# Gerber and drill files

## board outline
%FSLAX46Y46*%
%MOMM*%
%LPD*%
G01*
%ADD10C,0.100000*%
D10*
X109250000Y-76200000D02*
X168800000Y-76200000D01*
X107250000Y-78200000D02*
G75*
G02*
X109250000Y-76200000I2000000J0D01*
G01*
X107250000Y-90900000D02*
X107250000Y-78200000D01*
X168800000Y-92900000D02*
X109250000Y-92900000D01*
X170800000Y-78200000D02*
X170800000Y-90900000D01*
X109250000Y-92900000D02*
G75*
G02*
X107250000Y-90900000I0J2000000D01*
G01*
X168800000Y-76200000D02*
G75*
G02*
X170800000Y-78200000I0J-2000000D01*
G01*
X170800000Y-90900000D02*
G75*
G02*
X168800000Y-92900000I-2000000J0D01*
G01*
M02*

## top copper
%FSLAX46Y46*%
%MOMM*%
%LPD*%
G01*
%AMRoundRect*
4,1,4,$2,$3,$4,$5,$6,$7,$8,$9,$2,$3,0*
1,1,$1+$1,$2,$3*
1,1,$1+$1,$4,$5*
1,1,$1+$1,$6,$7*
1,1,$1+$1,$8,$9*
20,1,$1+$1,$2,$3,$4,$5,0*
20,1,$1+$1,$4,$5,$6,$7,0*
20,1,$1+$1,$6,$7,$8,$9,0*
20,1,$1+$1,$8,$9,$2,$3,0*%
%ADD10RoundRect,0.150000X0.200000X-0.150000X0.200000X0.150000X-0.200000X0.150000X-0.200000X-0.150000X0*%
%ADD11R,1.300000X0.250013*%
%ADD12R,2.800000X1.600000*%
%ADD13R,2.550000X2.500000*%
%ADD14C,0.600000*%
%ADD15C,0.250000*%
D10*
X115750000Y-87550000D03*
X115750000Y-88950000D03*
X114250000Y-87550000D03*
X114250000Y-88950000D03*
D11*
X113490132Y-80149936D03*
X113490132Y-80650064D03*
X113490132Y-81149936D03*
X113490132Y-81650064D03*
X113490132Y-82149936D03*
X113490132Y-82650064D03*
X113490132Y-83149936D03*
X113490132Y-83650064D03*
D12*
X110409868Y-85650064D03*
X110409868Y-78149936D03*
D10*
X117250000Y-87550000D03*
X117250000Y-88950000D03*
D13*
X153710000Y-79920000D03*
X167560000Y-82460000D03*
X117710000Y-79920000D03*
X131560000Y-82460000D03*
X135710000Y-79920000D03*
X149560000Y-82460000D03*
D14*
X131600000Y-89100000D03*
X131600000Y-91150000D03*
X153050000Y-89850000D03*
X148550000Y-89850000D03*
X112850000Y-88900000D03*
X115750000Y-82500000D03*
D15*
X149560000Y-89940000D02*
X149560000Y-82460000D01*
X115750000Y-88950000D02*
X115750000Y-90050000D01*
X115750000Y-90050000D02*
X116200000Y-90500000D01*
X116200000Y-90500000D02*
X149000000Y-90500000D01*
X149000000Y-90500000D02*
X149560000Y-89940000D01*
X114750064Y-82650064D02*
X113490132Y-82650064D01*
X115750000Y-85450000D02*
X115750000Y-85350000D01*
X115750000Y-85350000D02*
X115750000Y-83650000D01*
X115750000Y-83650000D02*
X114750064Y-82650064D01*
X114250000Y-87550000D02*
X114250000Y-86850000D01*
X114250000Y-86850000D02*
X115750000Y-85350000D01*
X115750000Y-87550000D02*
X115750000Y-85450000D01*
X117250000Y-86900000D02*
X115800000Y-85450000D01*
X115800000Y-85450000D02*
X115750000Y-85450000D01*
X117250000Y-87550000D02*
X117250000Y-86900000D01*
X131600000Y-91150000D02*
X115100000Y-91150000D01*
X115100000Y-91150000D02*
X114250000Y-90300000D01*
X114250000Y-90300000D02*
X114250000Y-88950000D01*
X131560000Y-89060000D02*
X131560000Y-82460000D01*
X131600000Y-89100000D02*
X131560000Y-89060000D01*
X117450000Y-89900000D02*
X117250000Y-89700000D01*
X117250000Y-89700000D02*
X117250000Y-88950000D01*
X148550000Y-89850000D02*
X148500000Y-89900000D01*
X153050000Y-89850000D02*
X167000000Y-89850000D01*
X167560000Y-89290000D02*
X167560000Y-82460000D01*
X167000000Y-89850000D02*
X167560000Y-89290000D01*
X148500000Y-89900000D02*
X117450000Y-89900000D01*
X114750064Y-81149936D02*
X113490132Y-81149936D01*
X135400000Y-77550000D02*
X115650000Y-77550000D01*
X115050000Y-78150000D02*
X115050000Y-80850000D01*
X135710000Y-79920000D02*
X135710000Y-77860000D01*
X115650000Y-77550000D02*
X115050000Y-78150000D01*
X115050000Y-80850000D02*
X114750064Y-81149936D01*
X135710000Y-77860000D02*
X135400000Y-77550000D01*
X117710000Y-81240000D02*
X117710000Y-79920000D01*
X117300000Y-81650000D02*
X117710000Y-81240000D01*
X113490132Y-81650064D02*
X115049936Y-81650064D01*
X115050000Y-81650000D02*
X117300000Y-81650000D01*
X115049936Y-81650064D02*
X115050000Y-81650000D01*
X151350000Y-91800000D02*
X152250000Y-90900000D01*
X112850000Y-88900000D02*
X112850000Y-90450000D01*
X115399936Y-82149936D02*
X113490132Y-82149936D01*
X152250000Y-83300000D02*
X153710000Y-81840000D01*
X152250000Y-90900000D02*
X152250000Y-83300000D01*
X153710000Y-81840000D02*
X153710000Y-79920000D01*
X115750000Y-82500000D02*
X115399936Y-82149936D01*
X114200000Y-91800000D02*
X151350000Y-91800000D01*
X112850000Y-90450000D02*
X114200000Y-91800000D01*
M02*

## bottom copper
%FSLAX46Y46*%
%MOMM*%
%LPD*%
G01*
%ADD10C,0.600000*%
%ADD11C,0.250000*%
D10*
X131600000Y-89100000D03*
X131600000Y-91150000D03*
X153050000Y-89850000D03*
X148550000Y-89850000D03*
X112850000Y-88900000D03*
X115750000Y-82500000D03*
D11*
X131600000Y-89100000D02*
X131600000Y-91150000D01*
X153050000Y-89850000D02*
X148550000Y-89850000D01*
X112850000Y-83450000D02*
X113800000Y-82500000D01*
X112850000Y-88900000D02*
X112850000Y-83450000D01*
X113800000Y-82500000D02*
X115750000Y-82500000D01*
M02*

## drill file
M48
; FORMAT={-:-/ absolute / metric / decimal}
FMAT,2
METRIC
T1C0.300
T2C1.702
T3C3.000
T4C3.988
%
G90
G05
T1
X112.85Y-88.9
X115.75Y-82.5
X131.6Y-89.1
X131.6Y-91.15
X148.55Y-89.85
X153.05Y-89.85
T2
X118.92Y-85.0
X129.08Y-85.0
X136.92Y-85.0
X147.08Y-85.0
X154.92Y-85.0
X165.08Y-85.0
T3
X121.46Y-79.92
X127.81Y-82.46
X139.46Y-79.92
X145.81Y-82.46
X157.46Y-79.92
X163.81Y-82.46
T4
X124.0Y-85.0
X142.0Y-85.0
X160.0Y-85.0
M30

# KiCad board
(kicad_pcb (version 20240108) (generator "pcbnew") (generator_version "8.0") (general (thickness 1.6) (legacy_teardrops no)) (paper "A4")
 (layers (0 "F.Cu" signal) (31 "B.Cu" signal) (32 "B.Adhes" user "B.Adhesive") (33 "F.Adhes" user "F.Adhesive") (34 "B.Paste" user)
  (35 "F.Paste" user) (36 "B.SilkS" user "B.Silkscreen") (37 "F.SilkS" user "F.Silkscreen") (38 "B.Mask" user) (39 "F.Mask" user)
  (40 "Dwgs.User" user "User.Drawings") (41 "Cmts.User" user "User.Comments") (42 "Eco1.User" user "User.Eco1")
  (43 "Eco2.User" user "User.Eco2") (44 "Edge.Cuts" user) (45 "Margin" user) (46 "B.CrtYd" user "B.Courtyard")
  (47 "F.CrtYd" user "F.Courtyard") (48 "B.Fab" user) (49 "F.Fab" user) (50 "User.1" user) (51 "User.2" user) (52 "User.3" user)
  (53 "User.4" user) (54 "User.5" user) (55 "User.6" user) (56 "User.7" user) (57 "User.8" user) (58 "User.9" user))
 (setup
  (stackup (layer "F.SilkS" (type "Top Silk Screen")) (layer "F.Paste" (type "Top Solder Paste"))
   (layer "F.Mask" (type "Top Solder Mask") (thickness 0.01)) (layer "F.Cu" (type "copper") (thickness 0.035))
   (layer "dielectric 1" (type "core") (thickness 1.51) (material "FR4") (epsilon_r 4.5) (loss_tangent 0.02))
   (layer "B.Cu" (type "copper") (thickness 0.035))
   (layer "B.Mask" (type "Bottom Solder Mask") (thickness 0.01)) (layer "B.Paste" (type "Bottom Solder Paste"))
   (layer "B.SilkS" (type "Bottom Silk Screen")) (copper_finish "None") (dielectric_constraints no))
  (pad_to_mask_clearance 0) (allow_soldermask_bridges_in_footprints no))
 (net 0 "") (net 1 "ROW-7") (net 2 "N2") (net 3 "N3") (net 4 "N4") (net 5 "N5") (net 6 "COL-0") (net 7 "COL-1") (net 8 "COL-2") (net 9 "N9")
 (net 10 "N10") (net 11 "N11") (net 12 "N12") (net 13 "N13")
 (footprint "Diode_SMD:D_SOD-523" (layer "F.Cu") (at 115.75 88.25 -90)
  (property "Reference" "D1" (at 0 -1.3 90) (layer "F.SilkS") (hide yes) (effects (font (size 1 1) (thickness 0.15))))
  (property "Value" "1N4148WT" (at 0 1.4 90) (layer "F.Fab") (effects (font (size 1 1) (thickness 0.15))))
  (pad "1" smd roundrect (at -0.7 0 90) (size 0.6 0.7) (layers "F.Cu" "F.Paste" "F.Mask") (roundrect_rratio 0.25) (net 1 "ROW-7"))
  (pad "2" smd roundrect (at 0.7 0 90) (size 0.6 0.7) (layers "F.Cu" "F.Paste" "F.Mask") (roundrect_rratio 0.25) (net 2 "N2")))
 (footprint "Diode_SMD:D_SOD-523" (layer "F.Cu") (at 114.25 88.25 -90)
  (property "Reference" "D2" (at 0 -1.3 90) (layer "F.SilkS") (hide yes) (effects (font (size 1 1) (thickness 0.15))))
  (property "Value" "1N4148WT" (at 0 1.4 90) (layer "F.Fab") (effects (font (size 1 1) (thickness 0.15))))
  (pad "1" smd roundrect (at -0.7 0 90) (size 0.6 0.7) (layers "F.Cu" "F.Paste" "F.Mask") (roundrect_rratio 0.25) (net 1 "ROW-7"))
  (pad "2" smd roundrect (at 0.7 0 90) (size 0.6 0.7) (layers "F.Cu" "F.Paste" "F.Mask") (roundrect_rratio 0.25) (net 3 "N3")))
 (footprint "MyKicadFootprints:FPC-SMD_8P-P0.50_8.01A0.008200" (layer "F.Cu") (at 111.95 81.9 -90)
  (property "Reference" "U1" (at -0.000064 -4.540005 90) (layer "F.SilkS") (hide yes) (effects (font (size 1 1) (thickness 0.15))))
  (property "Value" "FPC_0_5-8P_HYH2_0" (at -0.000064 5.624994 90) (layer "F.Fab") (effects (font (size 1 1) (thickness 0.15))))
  (pad "1" smd rect (at -1.750064 -1.540132 270) (size 0.250013 1.3) (layers "F.Cu" "F.Paste" "F.Mask") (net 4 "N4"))
  (pad "2" smd rect (at -1.249936 -1.540132 270) (size 0.250013 1.3) (layers "F.Cu" "F.Paste" "F.Mask") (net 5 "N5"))
  (pad "3" smd rect (at -0.750064 -1.540132 270) (size 0.250013 1.3) (layers "F.Cu" "F.Paste" "F.Mask") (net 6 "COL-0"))
  (pad "4" smd rect (at -0.249936 -1.540132 270) (size 0.250013 1.3) (layers "F.Cu" "F.Paste" "F.Mask") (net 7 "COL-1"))
  (pad "5" smd rect (at 0.249936 -1.540132 270) (size 0.250013 1.3) (layers "F.Cu" "F.Paste" "F.Mask") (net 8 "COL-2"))
  (pad "6" smd rect (at 0.750064 -1.540132 270) (size 0.250013 1.3) (layers "F.Cu" "F.Paste" "F.Mask") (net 1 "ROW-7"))
  (pad "7" smd rect (at 1.249936 -1.540132 270) (size 0.250013 1.3) (layers "F.Cu" "F.Paste" "F.Mask") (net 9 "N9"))
  (pad "8" smd rect (at 1.750064 -1.540132 270) (size 0.250013 1.3) (layers "F.Cu" "F.Paste" "F.Mask") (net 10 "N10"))
  (pad "9" smd rect (at 3.750064 1.540132 270) (size 1.6 2.8) (layers "F.Cu" "F.Paste" "F.Mask") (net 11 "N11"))
  (pad "10" smd rect (at -3.750064 1.540132 270) (size 1.6 2.8) (layers "F.Cu" "F.Paste" "F.Mask") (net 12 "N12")))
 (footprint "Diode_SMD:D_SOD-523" (layer "F.Cu") (at 117.25 88.25 -90)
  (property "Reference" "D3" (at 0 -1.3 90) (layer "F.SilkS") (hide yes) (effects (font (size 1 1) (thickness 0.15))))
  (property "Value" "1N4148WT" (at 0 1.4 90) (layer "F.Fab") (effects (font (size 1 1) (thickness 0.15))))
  (pad "1" smd roundrect (at -0.7 0 90) (size 0.6 0.7) (layers "F.Cu" "F.Paste" "F.Mask") (roundrect_rratio 0.25) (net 1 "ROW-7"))
  (pad "2" smd roundrect (at 0.7 0 90) (size 0.6 0.7) (layers "F.Cu" "F.Paste" "F.Mask") (roundrect_rratio 0.25) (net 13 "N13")))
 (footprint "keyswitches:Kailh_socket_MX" (layer "B.Cu") (at 160 85 180)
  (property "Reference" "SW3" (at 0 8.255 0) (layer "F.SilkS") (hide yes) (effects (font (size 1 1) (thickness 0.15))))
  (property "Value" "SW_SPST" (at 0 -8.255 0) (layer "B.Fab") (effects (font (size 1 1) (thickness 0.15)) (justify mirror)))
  (pad "" np_thru_hole circle (at -5.08 0 180) (size 1.7018 1.7018) (drill 1.7018) (layers "*.Cu" "*.Mask"))
  (pad "" np_thru_hole circle (at -3.81 2.54 180) (size 3 3) (drill 3) (layers "*.Cu" "*.Mask"))
  (pad "" np_thru_hole circle (at 0 0 180) (size 3.9878 3.9878) (drill 3.9878) (layers "*.Cu" "*.Mask"))
  (pad "" np_thru_hole circle (at 2.54 5.08 180) (size 3 3) (drill 3) (layers "*.Cu" "*.Mask"))
  (pad "" np_thru_hole circle (at 5.08 0 180) (size 1.7018 1.7018) (drill 1.7018) (layers "*.Cu" "*.Mask"))
  (pad "1" smd rect (at 6.29 5.08 180) (size 2.55 2.5) (layers "F.Cu" "F.Paste" "F.Mask") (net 8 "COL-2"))
  (pad "2" smd rect (at -7.56 2.54 180) (size 2.55 2.5) (layers "F.Cu" "F.Paste" "F.Mask") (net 13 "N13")))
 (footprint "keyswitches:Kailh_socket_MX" (layer "B.Cu") (at 124 85 180)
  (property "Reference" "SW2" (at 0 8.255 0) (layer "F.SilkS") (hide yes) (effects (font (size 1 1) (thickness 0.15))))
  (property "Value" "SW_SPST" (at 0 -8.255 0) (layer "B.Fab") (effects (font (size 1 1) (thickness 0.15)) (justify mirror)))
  (pad "" np_thru_hole circle (at -5.08 0 180) (size 1.7018 1.7018) (drill 1.7018) (layers "*.Cu" "*.Mask"))
  (pad "" np_thru_hole circle (at -3.81 2.54 180) (size 3 3) (drill 3) (layers "*.Cu" "*.Mask"))
  (pad "" np_thru_hole circle (at 0 0 180) (size 3.9878 3.9878) (drill 3.9878) (layers "*.Cu" "*.Mask"))
  (pad "" np_thru_hole circle (at 2.54 5.08 180) (size 3 3) (drill 3) (layers "*.Cu" "*.Mask"))
  (pad "" np_thru_hole circle (at 5.08 0 180) (size 1.7018 1.7018) (drill 1.7018) (layers "*.Cu" "*.Mask"))
  (pad "1" smd rect (at 6.29 5.08 180) (size 2.55 2.5) (layers "F.Cu" "F.Paste" "F.Mask") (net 7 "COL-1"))
  (pad "2" smd rect (at -7.56 2.54 180) (size 2.55 2.5) (layers "F.Cu" "F.Paste" "F.Mask") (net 3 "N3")))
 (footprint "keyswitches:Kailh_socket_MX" (layer "B.Cu") (at 142 85 180)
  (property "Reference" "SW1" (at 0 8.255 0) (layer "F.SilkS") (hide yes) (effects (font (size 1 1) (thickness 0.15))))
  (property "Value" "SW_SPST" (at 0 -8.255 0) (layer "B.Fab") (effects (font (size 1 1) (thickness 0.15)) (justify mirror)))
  (pad "" np_thru_hole circle (at -5.08 0 180) (size 1.7018 1.7018) (drill 1.7018) (layers "*.Cu" "*.Mask"))
  (pad "" np_thru_hole circle (at -3.81 2.54 180) (size 3 3) (drill 3) (layers "*.Cu" "*.Mask"))
  (pad "" np_thru_hole circle (at 0 0 180) (size 3.9878 3.9878) (drill 3.9878) (layers "*.Cu" "*.Mask"))
  (pad "" np_thru_hole circle (at 2.54 5.08 180) (size 3 3) (drill 3) (layers "*.Cu" "*.Mask"))
  (pad "" np_thru_hole circle (at 5.08 0 180) (size 1.7018 1.7018) (drill 1.7018) (layers "*.Cu" "*.Mask"))
  (pad "1" smd rect (at 6.29 5.08 180) (size 2.55 2.5) (layers "F.Cu" "F.Paste" "F.Mask") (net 6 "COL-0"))
  (pad "2" smd rect (at -7.56 2.54 180) (size 2.55 2.5) (layers "F.Cu" "F.Paste" "F.Mask") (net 2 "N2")))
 (gr_line (start 109.25 76.2) (end 168.8 76.2) (stroke (width 0.1) (type default)) (layer "Edge.Cuts"))
 (gr_arc (start 107.25 78.2) (mid 107.835786 76.785786) (end 109.25 76.2) (stroke (width 0.1) (type default)) (layer "Edge.Cuts"))
 (gr_line (start 107.25 90.9) (end 107.25 78.2) (stroke (width 0.1) (type default)) (layer "Edge.Cuts"))
 (gr_line (start 168.8 92.9) (end 109.25 92.9) (stroke (width 0.1) (type default)) (layer "Edge.Cuts"))
 (gr_line (start 170.8 78.2) (end 170.8 90.9) (stroke (width 0.1) (type default)) (layer "Edge.Cuts"))
 (gr_arc (start 109.25 92.9) (mid 107.835786 92.314214) (end 107.25 90.9) (stroke (width 0.1) (type default)) (layer "Edge.Cuts"))
 (gr_arc (start 168.8 76.2) (mid 170.214214 76.785786) (end 170.8 78.2) (stroke (width 0.1) (type default)) (layer "Edge.Cuts"))
 (gr_arc (start 170.8 90.9) (mid 170.214214 92.314214) (end 168.8 92.9) (stroke (width 0.1) (type default)) (layer "Edge.Cuts"))
 (segment (start 149.56 89.94) (end 149.56 82.46) (width 0.25) (layer "F.Cu") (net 2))
 (segment (start 115.75 88.95) (end 115.75 90.05) (width 0.25) (layer "F.Cu") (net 2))
 (segment (start 115.75 90.05) (end 116.2 90.5) (width 0.25) (layer "F.Cu") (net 2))
 (segment (start 116.2 90.5) (end 149 90.5) (width 0.25) (layer "F.Cu") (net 2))
 (segment (start 149 90.5) (end 149.56 89.94) (width 0.25) (layer "F.Cu") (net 2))
 (segment (start 114.750064 82.650064) (end 113.490132 82.650064) (width 0.25) (layer "F.Cu") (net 1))
 (segment (start 115.75 85.45) (end 115.75 85.35) (width 0.25) (layer "F.Cu") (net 1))
 (segment (start 115.75 85.35) (end 115.75 83.65) (width 0.25) (layer "F.Cu") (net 1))
 (segment (start 115.75 83.65) (end 114.750064 82.650064) (width 0.25) (layer "F.Cu") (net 1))
 (segment (start 114.25 87.55) (end 114.25 86.85) (width 0.25) (layer "F.Cu") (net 1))
 (segment (start 114.25 86.85) (end 115.75 85.35) (width 0.25) (layer "F.Cu") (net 1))
 (segment (start 115.75 87.55) (end 115.75 85.45) (width 0.25) (layer "F.Cu") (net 1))
 (segment (start 117.25 86.9) (end 115.8 85.45) (width 0.25) (layer "F.Cu") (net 1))
 (segment (start 115.8 85.45) (end 115.75 85.45) (width 0.25) (layer "F.Cu") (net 1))
 (segment (start 117.25 87.55) (end 117.25 86.9) (width 0.25) (layer "F.Cu") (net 1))
 (segment (start 131.6 91.15) (end 115.1 91.15) (width 0.25) (layer "F.Cu") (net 3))
 (segment (start 115.1 91.15) (end 114.25 90.3) (width 0.25) (layer "F.Cu") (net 3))
 (segment (start 114.25 90.3) (end 114.25 88.95) (width 0.25) (layer "F.Cu") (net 3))
 (segment (start 131.56 89.06) (end 131.56 82.46) (width 0.25) (layer "F.Cu") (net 3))
 (segment (start 131.6 89.1) (end 131.56 89.06) (width 0.25) (layer "F.Cu") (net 3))
 (via (at 131.6 89.1) (size 0.6) (drill 0.3) (layers "F.Cu" "B.Cu") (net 3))
 (via (at 131.6 91.15) (size 0.6) (drill 0.3) (layers "F.Cu" "B.Cu") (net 3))
 (segment (start 131.6 89.1) (end 131.6 91.15) (width 0.25) (layer "B.Cu") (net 3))
 (segment (start 117.45 89.9) (end 117.25 89.7) (width 0.25) (layer "F.Cu") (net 13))
 (segment (start 117.25 89.7) (end 117.25 88.95) (width 0.25) (layer "F.Cu") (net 13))
 (segment (start 148.55 89.85) (end 148.5 89.9) (width 0.25) (layer "F.Cu") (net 13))
 (segment (start 153.05 89.85) (end 167 89.85) (width 0.25) (layer "F.Cu") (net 13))
 (segment (start 167.56 89.29) (end 167.56 82.46) (width 0.25) (layer "F.Cu") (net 13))
 (segment (start 167 89.85) (end 167.56 89.29) (width 0.25) (layer "F.Cu") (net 13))
 (segment (start 148.5 89.9) (end 117.45 89.9) (width 0.25) (layer "F.Cu") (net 13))
 (via (at 153.05 89.85) (size 0.6) (drill 0.3) (layers "F.Cu" "B.Cu") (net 13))
 (via (at 148.55 89.85) (size 0.6) (drill 0.3) (layers "F.Cu" "B.Cu") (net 13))
 (segment (start 153.05 89.85) (end 148.55 89.85) (width 0.25) (layer "B.Cu") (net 13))
 (segment (start 114.750064 81.149936) (end 113.490132 81.149936) (width 0.25) (layer "F.Cu") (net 6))
 (segment (start 135.4 77.55) (end 115.65 77.55) (width 0.25) (layer "F.Cu") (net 6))
 (segment (start 115.05 78.15) (end 115.05 80.85) (width 0.25) (layer "F.Cu") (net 6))
 (segment (start 135.71 79.92) (end 135.71 77.86) (width 0.25) (layer "F.Cu") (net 6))
 (segment (start 115.65 77.55) (end 115.05 78.15) (width 0.25) (layer "F.Cu") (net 6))
 (segment (start 115.05 80.85) (end 114.750064 81.149936) (width 0.25) (layer "F.Cu") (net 6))
 (segment (start 135.71 77.86) (end 135.4 77.55) (width 0.25) (layer "F.Cu") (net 6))
 (segment (start 117.71 81.24) (end 117.71 79.92) (width 0.25) (layer "F.Cu") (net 7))
 (segment (start 117.3 81.65) (end 117.71 81.24) (width 0.25) (layer "F.Cu") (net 7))
 (segment (start 113.490132 81.650064) (end 115.049936 81.650064) (width 0.25) (layer "F.Cu") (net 7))
 (segment (start 115.05 81.65) (end 117.3 81.65) (width 0.25) (layer "F.Cu") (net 7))
 (segment (start 115.049936 81.650064) (end 115.05 81.65) (width 0.25) (layer "F.Cu") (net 7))
 (segment (start 151.35 91.8) (end 152.25 90.9) (width 0.25) (layer "F.Cu") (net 8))
 (segment (start 112.85 88.9) (end 112.85 90.45) (width 0.25) (layer "F.Cu") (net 8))
 (segment (start 115.399936 82.149936) (end 113.490132 82.149936) (width 0.25) (layer "F.Cu") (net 8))
 (segment (start 152.25 83.3) (end 153.71 81.84) (width 0.25) (layer "F.Cu") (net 8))
 (segment (start 152.25 90.9) (end 152.25 83.3) (width 0.25) (layer "F.Cu") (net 8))
 (segment (start 153.71 81.84) (end 153.71 79.92) (width 0.25) (layer "F.Cu") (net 8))
 (segment (start 115.75 82.5) (end 115.399936 82.149936) (width 0.25) (layer "F.Cu") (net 8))
 (segment (start 114.2 91.8) (end 151.35 91.8) (width 0.25) (layer "F.Cu") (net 8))
 (segment (start 112.85 90.45) (end 114.2 91.8) (width 0.25) (layer "F.Cu") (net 8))
 (via (at 112.85 88.9) (size 0.6) (drill 0.3) (layers "F.Cu" "B.Cu") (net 8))
 (via (at 115.75 82.5) (size 0.6) (drill 0.3) (layers "F.Cu" "B.Cu") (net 8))
 (segment (start 112.85 83.45) (end 113.8 82.5) (width 0.25) (layer "B.Cu") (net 8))
 (segment (start 112.85 88.9) (end 112.85 83.45) (width 0.25) (layer "B.Cu") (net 8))
 (segment (start 113.8 82.5) (end 115.75 82.5) (width 0.25) (layer "B.Cu") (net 8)))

